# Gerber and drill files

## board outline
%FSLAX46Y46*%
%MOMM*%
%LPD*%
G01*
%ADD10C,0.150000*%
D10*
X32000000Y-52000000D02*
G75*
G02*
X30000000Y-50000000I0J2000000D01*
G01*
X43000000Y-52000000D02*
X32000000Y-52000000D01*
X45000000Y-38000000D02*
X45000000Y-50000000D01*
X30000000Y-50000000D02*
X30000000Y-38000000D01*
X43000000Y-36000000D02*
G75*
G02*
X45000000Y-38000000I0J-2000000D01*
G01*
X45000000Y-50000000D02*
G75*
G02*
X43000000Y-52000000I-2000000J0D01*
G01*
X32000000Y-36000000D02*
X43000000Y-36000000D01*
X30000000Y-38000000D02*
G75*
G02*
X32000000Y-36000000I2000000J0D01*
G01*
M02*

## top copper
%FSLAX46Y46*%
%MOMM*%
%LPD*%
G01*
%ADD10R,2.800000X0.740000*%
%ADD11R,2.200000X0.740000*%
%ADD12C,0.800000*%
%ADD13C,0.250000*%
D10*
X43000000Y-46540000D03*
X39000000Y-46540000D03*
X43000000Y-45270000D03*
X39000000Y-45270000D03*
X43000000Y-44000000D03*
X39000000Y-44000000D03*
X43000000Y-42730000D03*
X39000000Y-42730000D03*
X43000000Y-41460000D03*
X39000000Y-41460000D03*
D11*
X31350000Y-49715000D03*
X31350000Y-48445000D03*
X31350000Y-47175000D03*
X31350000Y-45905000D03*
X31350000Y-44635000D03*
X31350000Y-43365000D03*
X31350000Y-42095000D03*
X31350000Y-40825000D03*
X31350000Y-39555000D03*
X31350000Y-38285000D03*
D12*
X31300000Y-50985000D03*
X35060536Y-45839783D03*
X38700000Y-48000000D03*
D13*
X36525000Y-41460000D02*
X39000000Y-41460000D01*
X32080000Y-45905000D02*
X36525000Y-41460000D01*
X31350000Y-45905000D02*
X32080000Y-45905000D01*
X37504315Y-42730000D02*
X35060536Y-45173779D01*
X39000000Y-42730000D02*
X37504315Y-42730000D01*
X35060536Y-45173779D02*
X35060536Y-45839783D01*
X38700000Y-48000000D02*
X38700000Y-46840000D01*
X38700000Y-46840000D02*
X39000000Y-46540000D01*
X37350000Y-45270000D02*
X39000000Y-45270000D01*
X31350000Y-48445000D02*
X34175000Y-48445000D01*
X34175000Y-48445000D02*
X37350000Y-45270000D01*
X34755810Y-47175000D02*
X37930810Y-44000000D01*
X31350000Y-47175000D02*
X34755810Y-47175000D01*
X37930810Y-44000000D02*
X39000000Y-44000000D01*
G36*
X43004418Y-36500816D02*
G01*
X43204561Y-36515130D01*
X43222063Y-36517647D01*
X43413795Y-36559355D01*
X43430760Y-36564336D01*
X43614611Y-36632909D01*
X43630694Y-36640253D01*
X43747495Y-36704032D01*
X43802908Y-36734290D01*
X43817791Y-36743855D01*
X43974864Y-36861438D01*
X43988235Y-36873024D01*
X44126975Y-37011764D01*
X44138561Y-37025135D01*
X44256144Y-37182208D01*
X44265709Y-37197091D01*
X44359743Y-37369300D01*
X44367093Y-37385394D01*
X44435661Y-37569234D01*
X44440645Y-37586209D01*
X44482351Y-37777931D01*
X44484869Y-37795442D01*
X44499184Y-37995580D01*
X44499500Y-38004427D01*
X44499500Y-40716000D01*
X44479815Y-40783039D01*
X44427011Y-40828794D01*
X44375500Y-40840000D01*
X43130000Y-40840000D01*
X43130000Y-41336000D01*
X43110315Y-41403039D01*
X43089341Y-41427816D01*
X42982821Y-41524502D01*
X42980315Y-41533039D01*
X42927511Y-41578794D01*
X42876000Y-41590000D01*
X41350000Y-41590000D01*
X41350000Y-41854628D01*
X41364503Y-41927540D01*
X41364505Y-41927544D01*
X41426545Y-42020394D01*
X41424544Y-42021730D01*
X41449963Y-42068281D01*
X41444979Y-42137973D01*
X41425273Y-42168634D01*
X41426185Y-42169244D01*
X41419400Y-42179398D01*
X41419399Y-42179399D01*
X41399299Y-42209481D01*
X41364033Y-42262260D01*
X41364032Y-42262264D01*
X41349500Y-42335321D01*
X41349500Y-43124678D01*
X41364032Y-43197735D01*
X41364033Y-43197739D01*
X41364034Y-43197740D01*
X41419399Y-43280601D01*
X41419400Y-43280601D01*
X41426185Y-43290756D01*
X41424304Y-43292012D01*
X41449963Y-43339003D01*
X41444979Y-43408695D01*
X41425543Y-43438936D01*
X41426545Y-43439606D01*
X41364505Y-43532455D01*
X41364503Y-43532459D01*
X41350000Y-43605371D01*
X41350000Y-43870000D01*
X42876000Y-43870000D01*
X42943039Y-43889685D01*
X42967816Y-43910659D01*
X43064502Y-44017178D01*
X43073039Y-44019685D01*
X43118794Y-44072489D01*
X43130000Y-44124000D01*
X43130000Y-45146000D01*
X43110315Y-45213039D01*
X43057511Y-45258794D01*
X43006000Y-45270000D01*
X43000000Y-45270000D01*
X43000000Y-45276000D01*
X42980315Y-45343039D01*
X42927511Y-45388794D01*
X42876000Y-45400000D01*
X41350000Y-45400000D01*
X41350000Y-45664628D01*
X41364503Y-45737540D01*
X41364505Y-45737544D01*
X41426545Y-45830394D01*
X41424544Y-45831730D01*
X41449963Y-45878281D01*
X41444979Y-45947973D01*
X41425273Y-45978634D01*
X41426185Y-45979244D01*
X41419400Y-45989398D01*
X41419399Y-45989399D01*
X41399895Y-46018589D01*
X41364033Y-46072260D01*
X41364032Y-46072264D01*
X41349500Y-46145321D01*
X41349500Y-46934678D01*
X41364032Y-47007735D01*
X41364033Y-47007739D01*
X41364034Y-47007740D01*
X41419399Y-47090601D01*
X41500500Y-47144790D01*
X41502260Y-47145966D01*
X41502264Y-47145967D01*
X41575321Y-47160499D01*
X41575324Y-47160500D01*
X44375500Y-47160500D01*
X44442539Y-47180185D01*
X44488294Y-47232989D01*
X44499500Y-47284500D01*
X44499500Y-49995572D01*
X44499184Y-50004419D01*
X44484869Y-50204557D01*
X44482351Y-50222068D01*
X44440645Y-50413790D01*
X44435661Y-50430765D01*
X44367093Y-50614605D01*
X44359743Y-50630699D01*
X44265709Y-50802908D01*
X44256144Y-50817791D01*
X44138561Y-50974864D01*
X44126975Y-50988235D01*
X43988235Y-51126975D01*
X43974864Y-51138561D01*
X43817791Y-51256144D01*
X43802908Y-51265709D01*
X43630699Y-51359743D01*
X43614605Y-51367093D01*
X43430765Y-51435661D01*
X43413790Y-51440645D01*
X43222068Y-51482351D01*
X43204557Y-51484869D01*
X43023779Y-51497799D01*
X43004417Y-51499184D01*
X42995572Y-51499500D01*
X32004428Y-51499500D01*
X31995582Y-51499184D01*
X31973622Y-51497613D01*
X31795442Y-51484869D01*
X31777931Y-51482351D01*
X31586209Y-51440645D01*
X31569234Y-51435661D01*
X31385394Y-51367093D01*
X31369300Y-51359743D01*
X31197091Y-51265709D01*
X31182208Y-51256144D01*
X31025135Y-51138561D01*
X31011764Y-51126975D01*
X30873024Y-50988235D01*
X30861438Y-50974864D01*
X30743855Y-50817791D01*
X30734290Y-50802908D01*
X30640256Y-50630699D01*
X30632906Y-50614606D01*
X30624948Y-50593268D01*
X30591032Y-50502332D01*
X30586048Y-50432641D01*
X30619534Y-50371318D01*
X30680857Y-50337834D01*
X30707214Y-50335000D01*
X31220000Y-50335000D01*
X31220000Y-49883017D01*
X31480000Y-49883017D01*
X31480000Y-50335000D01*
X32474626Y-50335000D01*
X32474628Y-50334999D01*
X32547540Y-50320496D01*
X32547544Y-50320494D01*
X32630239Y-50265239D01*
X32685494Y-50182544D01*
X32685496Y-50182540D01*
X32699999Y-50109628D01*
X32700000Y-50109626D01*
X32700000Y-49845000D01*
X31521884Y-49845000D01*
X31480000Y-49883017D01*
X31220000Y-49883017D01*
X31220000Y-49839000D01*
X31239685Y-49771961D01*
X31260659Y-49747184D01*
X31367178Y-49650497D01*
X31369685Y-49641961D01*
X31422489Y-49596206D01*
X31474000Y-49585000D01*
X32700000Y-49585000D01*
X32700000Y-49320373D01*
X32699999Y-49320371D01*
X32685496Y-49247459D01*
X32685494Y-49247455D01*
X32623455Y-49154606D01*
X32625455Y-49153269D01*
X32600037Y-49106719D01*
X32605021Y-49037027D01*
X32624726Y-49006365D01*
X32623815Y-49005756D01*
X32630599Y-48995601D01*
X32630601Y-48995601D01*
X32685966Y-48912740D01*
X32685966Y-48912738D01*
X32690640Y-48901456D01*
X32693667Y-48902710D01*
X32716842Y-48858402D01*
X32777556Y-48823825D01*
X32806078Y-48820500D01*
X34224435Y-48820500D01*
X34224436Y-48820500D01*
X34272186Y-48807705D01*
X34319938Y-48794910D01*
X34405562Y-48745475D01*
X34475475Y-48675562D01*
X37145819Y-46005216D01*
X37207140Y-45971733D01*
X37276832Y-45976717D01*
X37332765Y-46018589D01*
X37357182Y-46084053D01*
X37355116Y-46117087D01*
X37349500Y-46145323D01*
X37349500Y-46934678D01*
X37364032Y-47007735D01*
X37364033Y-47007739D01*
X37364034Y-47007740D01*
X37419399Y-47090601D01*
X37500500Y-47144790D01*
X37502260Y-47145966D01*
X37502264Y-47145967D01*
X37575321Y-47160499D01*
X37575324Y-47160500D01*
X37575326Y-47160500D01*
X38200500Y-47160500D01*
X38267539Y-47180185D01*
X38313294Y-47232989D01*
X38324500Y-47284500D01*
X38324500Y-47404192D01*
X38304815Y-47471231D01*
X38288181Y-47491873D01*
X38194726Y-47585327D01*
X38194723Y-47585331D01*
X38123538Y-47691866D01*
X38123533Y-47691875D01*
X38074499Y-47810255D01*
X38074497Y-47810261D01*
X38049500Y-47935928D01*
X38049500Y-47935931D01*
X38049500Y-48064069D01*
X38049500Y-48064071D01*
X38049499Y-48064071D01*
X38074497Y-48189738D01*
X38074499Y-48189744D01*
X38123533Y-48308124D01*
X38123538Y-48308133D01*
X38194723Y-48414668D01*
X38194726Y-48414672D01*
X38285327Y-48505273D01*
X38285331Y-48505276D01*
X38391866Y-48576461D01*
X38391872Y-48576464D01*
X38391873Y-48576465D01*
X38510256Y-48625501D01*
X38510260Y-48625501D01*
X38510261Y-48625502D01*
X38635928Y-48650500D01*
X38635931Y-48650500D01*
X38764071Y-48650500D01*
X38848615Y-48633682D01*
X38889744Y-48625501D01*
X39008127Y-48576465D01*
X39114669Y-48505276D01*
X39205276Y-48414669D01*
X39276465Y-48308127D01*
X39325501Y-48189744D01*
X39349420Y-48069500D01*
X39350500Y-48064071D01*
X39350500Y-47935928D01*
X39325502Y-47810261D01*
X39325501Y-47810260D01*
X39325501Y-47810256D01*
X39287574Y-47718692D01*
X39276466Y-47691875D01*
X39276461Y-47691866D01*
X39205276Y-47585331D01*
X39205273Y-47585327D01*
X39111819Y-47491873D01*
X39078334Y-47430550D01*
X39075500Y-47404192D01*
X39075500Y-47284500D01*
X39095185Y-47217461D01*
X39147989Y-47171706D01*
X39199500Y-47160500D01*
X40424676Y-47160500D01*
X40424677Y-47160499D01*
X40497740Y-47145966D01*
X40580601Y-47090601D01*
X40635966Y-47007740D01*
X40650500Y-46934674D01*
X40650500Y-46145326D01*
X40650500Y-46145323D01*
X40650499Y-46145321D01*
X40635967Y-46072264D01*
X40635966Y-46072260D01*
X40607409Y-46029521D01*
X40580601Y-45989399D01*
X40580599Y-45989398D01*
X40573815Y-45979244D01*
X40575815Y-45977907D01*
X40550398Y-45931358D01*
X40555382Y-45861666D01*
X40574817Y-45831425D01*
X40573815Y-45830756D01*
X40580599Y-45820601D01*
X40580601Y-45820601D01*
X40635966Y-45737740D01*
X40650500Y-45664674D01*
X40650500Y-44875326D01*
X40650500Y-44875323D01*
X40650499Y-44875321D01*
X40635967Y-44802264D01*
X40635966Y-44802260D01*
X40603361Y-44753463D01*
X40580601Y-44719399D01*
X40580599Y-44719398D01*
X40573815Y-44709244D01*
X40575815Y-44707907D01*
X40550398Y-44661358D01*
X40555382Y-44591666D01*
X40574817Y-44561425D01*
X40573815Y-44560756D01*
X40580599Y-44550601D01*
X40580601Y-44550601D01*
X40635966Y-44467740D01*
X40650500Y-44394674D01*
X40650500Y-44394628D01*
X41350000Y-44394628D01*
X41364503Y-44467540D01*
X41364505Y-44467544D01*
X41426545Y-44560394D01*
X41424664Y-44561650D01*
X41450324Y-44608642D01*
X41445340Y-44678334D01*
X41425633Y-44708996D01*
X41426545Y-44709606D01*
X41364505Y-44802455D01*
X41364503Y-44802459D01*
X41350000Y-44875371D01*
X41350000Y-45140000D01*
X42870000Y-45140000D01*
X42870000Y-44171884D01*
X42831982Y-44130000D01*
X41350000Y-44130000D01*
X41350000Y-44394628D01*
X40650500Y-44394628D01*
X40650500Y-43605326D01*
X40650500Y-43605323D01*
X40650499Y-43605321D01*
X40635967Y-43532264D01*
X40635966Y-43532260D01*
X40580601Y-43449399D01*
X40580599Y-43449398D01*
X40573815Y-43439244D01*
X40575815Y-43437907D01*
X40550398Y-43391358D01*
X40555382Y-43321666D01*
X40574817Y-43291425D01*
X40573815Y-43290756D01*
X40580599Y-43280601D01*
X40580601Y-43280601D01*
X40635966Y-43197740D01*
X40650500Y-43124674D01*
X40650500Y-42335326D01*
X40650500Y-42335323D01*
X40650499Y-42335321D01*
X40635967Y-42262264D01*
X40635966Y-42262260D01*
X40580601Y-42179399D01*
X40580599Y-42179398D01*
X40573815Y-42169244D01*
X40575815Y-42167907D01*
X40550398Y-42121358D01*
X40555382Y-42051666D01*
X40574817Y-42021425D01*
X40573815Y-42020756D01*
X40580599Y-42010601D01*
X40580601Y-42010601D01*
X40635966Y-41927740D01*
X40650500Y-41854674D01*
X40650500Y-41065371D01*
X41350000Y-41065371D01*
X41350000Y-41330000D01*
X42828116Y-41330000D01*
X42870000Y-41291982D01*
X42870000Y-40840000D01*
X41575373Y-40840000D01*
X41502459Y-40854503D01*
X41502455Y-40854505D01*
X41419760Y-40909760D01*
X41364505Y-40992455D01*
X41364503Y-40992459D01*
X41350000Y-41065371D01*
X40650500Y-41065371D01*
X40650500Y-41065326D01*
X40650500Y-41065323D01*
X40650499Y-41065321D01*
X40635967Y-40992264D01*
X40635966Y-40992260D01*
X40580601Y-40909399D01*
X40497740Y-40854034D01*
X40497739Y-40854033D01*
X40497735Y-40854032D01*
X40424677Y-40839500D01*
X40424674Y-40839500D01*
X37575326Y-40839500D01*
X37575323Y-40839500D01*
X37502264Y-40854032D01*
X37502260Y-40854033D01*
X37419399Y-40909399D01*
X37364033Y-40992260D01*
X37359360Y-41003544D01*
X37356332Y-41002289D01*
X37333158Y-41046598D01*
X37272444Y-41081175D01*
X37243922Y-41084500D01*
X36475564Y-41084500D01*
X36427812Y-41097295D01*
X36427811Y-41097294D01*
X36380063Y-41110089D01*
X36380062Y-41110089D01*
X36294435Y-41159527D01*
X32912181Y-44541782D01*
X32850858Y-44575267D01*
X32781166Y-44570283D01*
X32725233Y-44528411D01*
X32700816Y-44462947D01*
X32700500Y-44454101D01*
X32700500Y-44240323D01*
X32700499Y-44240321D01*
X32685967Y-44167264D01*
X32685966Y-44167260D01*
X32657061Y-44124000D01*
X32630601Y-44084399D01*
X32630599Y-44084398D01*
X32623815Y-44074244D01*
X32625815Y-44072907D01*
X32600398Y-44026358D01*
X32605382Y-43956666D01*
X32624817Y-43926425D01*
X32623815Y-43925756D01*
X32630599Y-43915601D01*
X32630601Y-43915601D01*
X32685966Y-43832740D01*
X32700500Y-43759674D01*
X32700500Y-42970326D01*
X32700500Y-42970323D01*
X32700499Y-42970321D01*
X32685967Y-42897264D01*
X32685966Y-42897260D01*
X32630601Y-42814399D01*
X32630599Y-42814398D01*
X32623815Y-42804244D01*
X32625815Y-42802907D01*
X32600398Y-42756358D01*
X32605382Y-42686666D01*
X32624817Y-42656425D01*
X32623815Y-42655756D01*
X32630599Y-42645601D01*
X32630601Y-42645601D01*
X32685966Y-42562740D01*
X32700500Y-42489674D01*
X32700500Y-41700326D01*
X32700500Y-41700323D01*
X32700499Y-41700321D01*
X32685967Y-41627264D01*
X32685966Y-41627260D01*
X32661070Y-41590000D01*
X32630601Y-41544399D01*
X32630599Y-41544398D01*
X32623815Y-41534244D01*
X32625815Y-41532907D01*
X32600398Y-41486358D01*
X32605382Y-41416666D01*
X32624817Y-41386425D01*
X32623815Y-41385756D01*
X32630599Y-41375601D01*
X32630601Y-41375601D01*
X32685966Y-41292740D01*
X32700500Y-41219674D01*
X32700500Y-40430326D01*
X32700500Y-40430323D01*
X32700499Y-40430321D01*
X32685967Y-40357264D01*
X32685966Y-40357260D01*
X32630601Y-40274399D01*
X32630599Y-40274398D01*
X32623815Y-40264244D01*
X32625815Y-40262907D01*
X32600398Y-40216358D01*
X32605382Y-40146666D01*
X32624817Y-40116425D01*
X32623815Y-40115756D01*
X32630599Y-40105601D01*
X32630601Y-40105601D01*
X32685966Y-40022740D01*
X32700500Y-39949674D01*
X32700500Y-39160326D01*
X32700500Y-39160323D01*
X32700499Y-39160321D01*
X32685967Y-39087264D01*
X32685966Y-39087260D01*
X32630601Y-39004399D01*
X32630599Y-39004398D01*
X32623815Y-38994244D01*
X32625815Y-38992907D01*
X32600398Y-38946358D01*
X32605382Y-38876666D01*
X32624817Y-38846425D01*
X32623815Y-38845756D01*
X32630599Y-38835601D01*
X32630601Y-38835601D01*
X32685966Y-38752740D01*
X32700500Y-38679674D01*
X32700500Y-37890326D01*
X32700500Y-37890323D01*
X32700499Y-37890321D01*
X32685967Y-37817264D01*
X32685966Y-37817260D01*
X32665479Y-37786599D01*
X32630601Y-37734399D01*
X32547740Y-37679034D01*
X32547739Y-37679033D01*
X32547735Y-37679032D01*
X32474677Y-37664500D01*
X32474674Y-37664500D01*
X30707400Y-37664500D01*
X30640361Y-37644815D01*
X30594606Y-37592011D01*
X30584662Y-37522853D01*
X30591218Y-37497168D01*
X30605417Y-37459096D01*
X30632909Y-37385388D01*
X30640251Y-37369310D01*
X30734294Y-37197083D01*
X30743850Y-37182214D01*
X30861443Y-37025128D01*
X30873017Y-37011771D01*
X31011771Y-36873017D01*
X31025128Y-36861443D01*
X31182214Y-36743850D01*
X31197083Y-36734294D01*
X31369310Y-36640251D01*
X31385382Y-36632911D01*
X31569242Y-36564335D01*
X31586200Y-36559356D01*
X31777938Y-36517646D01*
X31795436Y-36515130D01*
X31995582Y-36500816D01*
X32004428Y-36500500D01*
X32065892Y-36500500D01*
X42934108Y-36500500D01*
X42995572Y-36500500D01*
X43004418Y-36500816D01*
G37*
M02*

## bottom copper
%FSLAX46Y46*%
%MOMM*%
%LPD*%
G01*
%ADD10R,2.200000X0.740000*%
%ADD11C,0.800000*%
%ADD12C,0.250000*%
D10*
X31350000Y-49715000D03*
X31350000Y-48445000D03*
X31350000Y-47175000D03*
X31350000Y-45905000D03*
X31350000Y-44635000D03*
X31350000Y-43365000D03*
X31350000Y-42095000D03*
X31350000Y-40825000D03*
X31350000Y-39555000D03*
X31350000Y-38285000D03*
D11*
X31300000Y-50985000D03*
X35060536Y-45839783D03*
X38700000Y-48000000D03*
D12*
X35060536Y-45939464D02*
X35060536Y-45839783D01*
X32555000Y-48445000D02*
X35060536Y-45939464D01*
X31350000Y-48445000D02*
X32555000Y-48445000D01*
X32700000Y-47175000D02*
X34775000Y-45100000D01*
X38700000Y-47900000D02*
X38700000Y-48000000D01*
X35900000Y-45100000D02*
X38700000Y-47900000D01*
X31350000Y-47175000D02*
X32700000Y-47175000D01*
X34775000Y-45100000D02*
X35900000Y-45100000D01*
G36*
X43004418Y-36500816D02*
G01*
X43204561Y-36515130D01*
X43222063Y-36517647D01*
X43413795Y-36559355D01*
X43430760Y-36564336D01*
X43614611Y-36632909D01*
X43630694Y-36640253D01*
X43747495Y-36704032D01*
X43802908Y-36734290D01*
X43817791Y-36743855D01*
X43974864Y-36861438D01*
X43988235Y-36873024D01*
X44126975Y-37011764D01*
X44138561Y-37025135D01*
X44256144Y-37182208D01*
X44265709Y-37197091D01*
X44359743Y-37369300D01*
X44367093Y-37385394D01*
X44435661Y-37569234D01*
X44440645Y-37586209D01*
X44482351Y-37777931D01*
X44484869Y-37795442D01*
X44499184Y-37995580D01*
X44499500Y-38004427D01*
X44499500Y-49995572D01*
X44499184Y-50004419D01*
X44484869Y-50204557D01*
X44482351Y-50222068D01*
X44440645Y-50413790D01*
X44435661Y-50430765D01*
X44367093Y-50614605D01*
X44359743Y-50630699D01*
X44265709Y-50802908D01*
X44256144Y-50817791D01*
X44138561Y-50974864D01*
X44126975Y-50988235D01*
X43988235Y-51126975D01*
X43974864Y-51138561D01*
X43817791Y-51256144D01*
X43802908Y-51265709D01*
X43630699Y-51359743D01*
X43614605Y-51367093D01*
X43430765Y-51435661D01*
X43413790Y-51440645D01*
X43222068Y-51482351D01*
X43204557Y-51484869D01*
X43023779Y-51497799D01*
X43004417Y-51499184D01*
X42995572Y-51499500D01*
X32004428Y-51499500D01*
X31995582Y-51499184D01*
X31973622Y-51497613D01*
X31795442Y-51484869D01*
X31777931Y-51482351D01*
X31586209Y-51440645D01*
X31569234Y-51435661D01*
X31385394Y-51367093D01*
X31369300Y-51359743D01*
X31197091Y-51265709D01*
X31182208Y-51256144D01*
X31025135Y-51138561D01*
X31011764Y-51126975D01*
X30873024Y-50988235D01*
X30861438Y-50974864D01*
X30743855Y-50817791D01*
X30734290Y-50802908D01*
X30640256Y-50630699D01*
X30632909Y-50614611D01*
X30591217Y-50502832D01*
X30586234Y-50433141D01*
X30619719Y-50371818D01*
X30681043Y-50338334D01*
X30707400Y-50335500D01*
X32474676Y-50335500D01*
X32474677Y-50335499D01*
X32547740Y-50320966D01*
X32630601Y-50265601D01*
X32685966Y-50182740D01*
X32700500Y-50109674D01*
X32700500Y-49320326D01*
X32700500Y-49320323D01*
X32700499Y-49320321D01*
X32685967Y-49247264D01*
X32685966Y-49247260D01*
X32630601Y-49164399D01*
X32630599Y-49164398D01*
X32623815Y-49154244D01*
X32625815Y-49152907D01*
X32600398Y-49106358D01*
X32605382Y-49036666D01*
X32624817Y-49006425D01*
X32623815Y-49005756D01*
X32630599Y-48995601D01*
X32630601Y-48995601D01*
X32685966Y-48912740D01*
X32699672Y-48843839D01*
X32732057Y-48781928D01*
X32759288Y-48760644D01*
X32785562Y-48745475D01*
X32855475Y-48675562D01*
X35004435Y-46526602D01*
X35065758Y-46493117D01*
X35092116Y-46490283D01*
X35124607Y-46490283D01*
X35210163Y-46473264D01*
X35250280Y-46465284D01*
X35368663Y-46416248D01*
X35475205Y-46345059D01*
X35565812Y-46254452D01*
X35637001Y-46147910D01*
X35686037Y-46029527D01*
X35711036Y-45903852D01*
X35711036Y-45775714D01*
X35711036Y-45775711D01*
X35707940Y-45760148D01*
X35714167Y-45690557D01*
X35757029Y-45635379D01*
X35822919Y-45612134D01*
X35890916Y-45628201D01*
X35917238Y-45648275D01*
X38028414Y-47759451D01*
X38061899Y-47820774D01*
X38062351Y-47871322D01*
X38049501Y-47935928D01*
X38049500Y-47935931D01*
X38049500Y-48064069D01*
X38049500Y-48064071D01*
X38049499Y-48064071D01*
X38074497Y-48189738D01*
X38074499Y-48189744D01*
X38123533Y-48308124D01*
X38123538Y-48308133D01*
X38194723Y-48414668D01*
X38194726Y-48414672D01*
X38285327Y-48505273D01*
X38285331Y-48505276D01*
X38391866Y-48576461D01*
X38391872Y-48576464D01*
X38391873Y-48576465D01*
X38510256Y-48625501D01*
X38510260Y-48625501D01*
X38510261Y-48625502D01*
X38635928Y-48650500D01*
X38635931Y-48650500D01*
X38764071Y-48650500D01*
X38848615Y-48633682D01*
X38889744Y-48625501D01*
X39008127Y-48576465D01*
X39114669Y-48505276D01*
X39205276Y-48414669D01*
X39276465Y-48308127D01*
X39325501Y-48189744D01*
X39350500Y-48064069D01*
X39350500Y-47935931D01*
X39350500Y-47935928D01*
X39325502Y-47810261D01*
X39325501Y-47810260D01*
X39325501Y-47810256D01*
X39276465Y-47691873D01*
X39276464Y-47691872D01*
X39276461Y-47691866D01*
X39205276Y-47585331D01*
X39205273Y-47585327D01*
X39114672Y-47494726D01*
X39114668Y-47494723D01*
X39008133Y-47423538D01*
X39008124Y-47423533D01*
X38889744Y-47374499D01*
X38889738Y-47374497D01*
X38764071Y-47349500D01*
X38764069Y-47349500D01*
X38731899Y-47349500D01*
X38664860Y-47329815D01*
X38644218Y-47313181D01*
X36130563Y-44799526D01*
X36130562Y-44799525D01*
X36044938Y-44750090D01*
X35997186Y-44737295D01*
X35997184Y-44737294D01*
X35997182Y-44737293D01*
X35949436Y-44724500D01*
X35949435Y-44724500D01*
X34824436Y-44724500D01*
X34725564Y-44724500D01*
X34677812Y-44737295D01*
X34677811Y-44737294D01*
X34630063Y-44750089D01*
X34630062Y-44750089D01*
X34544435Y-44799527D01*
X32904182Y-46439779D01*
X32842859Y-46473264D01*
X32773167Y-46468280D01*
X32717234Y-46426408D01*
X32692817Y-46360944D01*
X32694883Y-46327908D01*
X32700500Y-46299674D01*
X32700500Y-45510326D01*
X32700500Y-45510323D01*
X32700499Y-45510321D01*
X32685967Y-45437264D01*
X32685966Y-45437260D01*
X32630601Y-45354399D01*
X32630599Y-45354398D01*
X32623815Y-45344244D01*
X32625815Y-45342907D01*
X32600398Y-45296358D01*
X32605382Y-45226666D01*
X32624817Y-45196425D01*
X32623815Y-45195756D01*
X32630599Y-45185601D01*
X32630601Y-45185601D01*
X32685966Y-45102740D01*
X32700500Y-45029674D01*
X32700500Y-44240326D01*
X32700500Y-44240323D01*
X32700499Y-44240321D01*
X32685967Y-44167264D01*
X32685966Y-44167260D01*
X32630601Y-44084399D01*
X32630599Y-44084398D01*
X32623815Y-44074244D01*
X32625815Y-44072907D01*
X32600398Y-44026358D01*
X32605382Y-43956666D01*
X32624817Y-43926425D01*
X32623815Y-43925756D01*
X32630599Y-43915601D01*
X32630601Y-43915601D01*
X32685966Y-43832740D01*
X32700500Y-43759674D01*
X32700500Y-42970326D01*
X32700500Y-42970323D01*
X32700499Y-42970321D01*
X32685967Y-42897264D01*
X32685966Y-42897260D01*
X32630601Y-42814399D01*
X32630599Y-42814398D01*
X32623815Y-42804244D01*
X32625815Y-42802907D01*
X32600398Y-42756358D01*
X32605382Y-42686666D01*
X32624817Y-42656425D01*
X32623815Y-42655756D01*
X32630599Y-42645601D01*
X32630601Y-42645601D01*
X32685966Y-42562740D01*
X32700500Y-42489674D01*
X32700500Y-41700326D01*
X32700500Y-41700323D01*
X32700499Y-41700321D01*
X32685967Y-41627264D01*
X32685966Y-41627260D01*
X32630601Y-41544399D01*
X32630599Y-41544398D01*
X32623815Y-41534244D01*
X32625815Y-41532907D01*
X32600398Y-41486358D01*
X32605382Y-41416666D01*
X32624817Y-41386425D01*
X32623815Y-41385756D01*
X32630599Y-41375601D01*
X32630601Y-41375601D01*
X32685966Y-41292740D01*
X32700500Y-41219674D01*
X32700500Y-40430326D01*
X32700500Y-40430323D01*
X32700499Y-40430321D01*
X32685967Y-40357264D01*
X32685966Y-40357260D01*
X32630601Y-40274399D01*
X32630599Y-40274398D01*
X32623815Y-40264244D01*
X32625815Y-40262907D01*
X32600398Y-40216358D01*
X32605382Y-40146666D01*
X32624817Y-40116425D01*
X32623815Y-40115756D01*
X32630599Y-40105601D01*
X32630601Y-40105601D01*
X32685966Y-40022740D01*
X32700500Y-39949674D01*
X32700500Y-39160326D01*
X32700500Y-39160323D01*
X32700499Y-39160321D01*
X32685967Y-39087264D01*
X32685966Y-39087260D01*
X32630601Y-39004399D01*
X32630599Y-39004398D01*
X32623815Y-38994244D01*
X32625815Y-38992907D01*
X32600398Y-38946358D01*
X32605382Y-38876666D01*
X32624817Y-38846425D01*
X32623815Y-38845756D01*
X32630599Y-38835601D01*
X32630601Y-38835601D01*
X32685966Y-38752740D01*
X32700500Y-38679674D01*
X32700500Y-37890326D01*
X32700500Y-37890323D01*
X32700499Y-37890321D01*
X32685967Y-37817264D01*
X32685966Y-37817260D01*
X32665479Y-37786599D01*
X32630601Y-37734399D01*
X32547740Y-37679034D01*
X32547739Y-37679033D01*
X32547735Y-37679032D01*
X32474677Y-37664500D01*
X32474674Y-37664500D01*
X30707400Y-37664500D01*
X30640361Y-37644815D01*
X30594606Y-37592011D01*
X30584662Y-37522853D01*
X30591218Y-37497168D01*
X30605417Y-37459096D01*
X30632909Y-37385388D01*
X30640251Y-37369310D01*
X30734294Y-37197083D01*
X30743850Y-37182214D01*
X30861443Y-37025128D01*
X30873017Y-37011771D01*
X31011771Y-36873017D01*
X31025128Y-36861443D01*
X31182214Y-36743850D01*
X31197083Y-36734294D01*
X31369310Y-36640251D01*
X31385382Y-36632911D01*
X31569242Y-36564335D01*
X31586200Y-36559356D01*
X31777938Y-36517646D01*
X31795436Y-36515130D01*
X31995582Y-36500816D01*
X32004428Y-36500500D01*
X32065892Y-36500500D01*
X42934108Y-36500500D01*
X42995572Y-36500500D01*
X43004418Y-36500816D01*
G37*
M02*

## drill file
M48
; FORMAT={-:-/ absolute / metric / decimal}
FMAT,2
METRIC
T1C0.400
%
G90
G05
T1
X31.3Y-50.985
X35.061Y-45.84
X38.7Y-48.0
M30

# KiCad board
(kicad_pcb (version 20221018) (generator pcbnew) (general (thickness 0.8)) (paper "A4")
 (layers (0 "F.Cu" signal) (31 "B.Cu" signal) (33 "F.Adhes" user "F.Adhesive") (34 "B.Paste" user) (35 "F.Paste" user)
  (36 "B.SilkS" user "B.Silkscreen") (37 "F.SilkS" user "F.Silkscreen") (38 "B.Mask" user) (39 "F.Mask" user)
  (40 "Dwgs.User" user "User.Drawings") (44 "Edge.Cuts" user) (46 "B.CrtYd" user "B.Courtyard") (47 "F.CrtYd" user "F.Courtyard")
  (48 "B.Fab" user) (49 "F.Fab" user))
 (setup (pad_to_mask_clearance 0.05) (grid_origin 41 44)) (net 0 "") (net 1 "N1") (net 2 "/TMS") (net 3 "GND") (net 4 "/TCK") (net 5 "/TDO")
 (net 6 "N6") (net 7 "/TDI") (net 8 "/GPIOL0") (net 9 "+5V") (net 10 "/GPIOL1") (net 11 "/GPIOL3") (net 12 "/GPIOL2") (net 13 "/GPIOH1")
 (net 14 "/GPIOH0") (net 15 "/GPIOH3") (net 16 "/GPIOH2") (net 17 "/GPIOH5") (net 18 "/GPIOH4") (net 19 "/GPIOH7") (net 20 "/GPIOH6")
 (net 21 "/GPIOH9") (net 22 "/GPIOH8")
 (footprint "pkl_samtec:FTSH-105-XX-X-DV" (layer "F.Cu") (at 41 44 -90)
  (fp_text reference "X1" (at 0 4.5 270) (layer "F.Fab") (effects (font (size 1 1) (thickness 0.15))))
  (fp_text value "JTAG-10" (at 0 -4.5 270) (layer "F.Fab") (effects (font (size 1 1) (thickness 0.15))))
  (pad "1" smd rect (at 2.54 -2 90) (size 0.74 2.8) (layers "F.Cu" "F.Paste" "F.Mask") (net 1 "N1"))
  (pad "2" smd rect (at 2.54 2 90) (size 0.74 2.8) (layers "F.Cu" "F.Paste" "F.Mask") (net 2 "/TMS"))
  (pad "3" smd rect (at 1.27 -2 90) (size 0.74 2.8) (layers "F.Cu" "F.Paste" "F.Mask") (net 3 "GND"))
  (pad "4" smd rect (at 1.27 2 90) (size 0.74 2.8) (layers "F.Cu" "F.Paste" "F.Mask") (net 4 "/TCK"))
  (pad "5" smd rect (at 0 -2 90) (size 0.74 2.8) (layers "F.Cu" "F.Paste" "F.Mask") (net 3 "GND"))
  (pad "6" smd rect (at 0 2 90) (size 0.74 2.8) (layers "F.Cu" "F.Paste" "F.Mask") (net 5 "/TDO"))
  (pad "7" smd rect (at -1.27 -2 90) (size 0.74 2.8) (layers "F.Cu" "F.Paste" "F.Mask") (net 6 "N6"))
  (pad "8" smd rect (at -1.27 2 90) (size 0.74 2.8) (layers "F.Cu" "F.Paste" "F.Mask") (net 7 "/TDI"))
  (pad "9" smd rect (at -2.54 -2 90) (size 0.74 2.8) (layers "F.Cu" "F.Paste" "F.Mask") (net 3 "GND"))
  (pad "10" smd rect (at -2.54 2 90) (size 0.74 2.8) (layers "F.Cu" "F.Paste" "F.Mask") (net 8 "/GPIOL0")))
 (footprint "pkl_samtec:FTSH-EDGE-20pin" (layer "B.Cu") (at 30 44 90)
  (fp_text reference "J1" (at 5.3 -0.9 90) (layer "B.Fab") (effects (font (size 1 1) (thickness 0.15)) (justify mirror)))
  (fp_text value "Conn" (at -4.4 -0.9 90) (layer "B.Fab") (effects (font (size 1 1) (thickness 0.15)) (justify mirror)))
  (pad "1" smd rect (at -5.715 1.35 90) (size 0.74 2.2) (layers "B.Cu" "B.Paste" "B.Mask") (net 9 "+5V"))
  (pad "2" smd rect (at -5.715 1.35 90) (size 0.74 2.2) (layers "F.Cu" "F.Paste" "F.Mask") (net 3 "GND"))
  (pad "3" smd rect (at -4.445 1.35 90) (size 0.74 2.2) (layers "B.Cu" "B.Paste" "B.Mask") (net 7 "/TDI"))
  (pad "4" smd rect (at -4.445 1.35 90) (size 0.74 2.2) (layers "F.Cu" "F.Paste" "F.Mask") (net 4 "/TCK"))
  (pad "5" smd rect (at -3.175 1.35 90) (size 0.74 2.2) (layers "B.Cu" "B.Paste" "B.Mask") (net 2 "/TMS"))
  (pad "6" smd rect (at -3.175 1.35 90) (size 0.74 2.2) (layers "F.Cu" "F.Paste" "F.Mask") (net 5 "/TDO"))
  (pad "7" smd rect (at -1.905 1.35 90) (size 0.74 2.2) (layers "B.Cu" "B.Paste" "B.Mask") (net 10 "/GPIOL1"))
  (pad "8" smd rect (at -1.905 1.35 90) (size 0.74 2.2) (layers "F.Cu" "F.Paste" "F.Mask") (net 8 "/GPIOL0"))
  (pad "9" smd rect (at -0.635 1.35 90) (size 0.74 2.2) (layers "B.Cu" "B.Paste" "B.Mask") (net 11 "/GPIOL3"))
  (pad "10" smd rect (at -0.635 1.35 90) (size 0.74 2.2) (layers "F.Cu" "F.Paste" "F.Mask") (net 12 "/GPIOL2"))
  (pad "11" smd rect (at 0.635 1.35 90) (size 0.74 2.2) (layers "B.Cu" "B.Paste" "B.Mask") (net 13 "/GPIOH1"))
  (pad "12" smd rect (at 0.635 1.35 90) (size 0.74 2.2) (layers "F.Cu" "F.Paste" "F.Mask") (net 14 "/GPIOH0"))
  (pad "13" smd rect (at 1.905 1.35 90) (size 0.74 2.2) (layers "B.Cu" "B.Paste" "B.Mask") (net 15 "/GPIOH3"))
  (pad "14" smd rect (at 1.905 1.35 90) (size 0.74 2.2) (layers "F.Cu" "F.Paste" "F.Mask") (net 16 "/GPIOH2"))
  (pad "15" smd rect (at 3.175 1.35 90) (size 0.74 2.2) (layers "B.Cu" "B.Paste" "B.Mask") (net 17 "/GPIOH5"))
  (pad "16" smd rect (at 3.175 1.35 90) (size 0.74 2.2) (layers "F.Cu" "F.Paste" "F.Mask") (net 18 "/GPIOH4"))
  (pad "17" smd rect (at 4.445 1.35 90) (size 0.74 2.2) (layers "B.Cu" "B.Paste" "B.Mask") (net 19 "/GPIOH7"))
  (pad "18" smd rect (at 4.445 1.35 90) (size 0.74 2.2) (layers "F.Cu" "F.Paste" "F.Mask") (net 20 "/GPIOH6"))
  (pad "19" smd rect (at 5.715 1.35 90) (size 0.74 2.2) (layers "B.Cu" "B.Paste" "B.Mask") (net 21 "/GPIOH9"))
  (pad "20" smd rect (at 5.715 1.35 90) (size 0.74 2.2) (layers "F.Cu" "F.Paste" "F.Mask") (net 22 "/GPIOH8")))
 (gr_arc (start 32 52) (mid 30.585786 51.414214) (end 30 50) (stroke (width 0.15) (type solid)) (layer "Edge.Cuts"))
 (gr_line (start 43 52) (end 32 52) (stroke (width 0.15) (type solid)) (layer "Edge.Cuts"))
 (gr_line (start 45 38) (end 45 50) (stroke (width 0.15) (type solid)) (layer "Edge.Cuts"))
 (gr_line (start 30 50) (end 30 38) (stroke (width 0.15) (type solid)) (layer "Edge.Cuts"))
 (gr_arc (start 43 36) (mid 44.414214 36.585786) (end 45 38) (stroke (width 0.15) (type solid)) (layer "Edge.Cuts"))
 (gr_arc (start 45 50) (mid 44.414214 51.414214) (end 43 52) (stroke (width 0.15) (type solid)) (layer "Edge.Cuts"))
 (gr_line (start 32 36) (end 43 36) (stroke (width 0.15) (type solid)) (layer "Edge.Cuts"))
 (gr_arc (start 30 38) (mid 30.585786 36.585786) (end 32 36) (stroke (width 0.15) (type solid)) (layer "Edge.Cuts"))
 (via (at 31.3 50.985) (size 0.8) (drill 0.4) (layers "F.Cu" "B.Cu") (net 3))
 (segment (start 36.525 41.46) (end 39 41.46) (width 0.25) (layer "F.Cu") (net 8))
 (segment (start 32.08 45.905) (end 36.525 41.46) (width 0.25) (layer "F.Cu") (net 8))
 (segment (start 31.35 45.905) (end 32.08 45.905) (width 0.25) (layer "F.Cu") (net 8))
 (segment (start 37.504315 42.73) (end 35.060536 45.173779) (width 0.25) (layer "F.Cu") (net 7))
 (segment (start 39 42.73) (end 37.504315 42.73) (width 0.25) (layer "F.Cu") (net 7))
 (segment (start 35.060536 45.173779) (end 35.060536 45.839783) (width 0.25) (layer "F.Cu") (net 7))
 (via (at 35.060536 45.839783) (size 0.8) (drill 0.4) (layers "F.Cu" "B.Cu") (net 7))
 (segment (start 35.060536 45.939464) (end 35.060536 45.839783) (width 0.25) (layer "B.Cu") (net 7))
 (segment (start 32.555 48.445) (end 35.060536 45.939464) (width 0.25) (layer "B.Cu") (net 7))
 (segment (start 31.35 48.445) (end 32.555 48.445) (width 0.25) (layer "B.Cu") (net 7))
 (segment (start 38.7 48) (end 38.7 46.84) (width 0.25) (layer "F.Cu") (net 2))
 (segment (start 38.7 46.84) (end 39 46.54) (width 0.25) (layer "F.Cu") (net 2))
 (via (at 38.7 48) (size 0.8) (drill 0.4) (layers "F.Cu" "B.Cu") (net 2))
 (segment (start 32.7 47.175) (end 34.775 45.1) (width 0.25) (layer "B.Cu") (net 2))
 (segment (start 38.7 47.9) (end 38.7 48) (width 0.25) (layer "B.Cu") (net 2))
 (segment (start 35.9 45.1) (end 38.7 47.9) (width 0.25) (layer "B.Cu") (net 2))
 (segment (start 31.35 47.175) (end 32.7 47.175) (width 0.25) (layer "B.Cu") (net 2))
 (segment (start 34.775 45.1) (end 35.9 45.1) (width 0.25) (layer "B.Cu") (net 2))
 (segment (start 37.35 45.27) (end 39 45.27) (width 0.25) (layer "F.Cu") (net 4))
 (segment (start 31.35 48.445) (end 34.175 48.445) (width 0.25) (layer "F.Cu") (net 4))
 (segment (start 34.175 48.445) (end 37.35 45.27) (width 0.25) (layer "F.Cu") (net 4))
 (segment (start 34.75581 47.175) (end 37.93081 44) (width 0.25) (layer "F.Cu") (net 5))
 (segment (start 31.35 47.175) (end 34.75581 47.175) (width 0.25) (layer "F.Cu") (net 5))
 (segment (start 37.93081 44) (end 39 44) (width 0.25) (layer "F.Cu") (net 5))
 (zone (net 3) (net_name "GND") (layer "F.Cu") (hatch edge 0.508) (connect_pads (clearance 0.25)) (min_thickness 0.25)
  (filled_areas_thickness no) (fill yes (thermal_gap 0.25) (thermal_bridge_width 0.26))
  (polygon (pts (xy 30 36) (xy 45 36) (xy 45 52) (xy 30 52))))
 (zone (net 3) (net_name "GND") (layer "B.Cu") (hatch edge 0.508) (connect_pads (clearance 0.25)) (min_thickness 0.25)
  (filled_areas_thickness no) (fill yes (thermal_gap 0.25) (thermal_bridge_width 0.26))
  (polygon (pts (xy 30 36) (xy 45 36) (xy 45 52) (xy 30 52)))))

